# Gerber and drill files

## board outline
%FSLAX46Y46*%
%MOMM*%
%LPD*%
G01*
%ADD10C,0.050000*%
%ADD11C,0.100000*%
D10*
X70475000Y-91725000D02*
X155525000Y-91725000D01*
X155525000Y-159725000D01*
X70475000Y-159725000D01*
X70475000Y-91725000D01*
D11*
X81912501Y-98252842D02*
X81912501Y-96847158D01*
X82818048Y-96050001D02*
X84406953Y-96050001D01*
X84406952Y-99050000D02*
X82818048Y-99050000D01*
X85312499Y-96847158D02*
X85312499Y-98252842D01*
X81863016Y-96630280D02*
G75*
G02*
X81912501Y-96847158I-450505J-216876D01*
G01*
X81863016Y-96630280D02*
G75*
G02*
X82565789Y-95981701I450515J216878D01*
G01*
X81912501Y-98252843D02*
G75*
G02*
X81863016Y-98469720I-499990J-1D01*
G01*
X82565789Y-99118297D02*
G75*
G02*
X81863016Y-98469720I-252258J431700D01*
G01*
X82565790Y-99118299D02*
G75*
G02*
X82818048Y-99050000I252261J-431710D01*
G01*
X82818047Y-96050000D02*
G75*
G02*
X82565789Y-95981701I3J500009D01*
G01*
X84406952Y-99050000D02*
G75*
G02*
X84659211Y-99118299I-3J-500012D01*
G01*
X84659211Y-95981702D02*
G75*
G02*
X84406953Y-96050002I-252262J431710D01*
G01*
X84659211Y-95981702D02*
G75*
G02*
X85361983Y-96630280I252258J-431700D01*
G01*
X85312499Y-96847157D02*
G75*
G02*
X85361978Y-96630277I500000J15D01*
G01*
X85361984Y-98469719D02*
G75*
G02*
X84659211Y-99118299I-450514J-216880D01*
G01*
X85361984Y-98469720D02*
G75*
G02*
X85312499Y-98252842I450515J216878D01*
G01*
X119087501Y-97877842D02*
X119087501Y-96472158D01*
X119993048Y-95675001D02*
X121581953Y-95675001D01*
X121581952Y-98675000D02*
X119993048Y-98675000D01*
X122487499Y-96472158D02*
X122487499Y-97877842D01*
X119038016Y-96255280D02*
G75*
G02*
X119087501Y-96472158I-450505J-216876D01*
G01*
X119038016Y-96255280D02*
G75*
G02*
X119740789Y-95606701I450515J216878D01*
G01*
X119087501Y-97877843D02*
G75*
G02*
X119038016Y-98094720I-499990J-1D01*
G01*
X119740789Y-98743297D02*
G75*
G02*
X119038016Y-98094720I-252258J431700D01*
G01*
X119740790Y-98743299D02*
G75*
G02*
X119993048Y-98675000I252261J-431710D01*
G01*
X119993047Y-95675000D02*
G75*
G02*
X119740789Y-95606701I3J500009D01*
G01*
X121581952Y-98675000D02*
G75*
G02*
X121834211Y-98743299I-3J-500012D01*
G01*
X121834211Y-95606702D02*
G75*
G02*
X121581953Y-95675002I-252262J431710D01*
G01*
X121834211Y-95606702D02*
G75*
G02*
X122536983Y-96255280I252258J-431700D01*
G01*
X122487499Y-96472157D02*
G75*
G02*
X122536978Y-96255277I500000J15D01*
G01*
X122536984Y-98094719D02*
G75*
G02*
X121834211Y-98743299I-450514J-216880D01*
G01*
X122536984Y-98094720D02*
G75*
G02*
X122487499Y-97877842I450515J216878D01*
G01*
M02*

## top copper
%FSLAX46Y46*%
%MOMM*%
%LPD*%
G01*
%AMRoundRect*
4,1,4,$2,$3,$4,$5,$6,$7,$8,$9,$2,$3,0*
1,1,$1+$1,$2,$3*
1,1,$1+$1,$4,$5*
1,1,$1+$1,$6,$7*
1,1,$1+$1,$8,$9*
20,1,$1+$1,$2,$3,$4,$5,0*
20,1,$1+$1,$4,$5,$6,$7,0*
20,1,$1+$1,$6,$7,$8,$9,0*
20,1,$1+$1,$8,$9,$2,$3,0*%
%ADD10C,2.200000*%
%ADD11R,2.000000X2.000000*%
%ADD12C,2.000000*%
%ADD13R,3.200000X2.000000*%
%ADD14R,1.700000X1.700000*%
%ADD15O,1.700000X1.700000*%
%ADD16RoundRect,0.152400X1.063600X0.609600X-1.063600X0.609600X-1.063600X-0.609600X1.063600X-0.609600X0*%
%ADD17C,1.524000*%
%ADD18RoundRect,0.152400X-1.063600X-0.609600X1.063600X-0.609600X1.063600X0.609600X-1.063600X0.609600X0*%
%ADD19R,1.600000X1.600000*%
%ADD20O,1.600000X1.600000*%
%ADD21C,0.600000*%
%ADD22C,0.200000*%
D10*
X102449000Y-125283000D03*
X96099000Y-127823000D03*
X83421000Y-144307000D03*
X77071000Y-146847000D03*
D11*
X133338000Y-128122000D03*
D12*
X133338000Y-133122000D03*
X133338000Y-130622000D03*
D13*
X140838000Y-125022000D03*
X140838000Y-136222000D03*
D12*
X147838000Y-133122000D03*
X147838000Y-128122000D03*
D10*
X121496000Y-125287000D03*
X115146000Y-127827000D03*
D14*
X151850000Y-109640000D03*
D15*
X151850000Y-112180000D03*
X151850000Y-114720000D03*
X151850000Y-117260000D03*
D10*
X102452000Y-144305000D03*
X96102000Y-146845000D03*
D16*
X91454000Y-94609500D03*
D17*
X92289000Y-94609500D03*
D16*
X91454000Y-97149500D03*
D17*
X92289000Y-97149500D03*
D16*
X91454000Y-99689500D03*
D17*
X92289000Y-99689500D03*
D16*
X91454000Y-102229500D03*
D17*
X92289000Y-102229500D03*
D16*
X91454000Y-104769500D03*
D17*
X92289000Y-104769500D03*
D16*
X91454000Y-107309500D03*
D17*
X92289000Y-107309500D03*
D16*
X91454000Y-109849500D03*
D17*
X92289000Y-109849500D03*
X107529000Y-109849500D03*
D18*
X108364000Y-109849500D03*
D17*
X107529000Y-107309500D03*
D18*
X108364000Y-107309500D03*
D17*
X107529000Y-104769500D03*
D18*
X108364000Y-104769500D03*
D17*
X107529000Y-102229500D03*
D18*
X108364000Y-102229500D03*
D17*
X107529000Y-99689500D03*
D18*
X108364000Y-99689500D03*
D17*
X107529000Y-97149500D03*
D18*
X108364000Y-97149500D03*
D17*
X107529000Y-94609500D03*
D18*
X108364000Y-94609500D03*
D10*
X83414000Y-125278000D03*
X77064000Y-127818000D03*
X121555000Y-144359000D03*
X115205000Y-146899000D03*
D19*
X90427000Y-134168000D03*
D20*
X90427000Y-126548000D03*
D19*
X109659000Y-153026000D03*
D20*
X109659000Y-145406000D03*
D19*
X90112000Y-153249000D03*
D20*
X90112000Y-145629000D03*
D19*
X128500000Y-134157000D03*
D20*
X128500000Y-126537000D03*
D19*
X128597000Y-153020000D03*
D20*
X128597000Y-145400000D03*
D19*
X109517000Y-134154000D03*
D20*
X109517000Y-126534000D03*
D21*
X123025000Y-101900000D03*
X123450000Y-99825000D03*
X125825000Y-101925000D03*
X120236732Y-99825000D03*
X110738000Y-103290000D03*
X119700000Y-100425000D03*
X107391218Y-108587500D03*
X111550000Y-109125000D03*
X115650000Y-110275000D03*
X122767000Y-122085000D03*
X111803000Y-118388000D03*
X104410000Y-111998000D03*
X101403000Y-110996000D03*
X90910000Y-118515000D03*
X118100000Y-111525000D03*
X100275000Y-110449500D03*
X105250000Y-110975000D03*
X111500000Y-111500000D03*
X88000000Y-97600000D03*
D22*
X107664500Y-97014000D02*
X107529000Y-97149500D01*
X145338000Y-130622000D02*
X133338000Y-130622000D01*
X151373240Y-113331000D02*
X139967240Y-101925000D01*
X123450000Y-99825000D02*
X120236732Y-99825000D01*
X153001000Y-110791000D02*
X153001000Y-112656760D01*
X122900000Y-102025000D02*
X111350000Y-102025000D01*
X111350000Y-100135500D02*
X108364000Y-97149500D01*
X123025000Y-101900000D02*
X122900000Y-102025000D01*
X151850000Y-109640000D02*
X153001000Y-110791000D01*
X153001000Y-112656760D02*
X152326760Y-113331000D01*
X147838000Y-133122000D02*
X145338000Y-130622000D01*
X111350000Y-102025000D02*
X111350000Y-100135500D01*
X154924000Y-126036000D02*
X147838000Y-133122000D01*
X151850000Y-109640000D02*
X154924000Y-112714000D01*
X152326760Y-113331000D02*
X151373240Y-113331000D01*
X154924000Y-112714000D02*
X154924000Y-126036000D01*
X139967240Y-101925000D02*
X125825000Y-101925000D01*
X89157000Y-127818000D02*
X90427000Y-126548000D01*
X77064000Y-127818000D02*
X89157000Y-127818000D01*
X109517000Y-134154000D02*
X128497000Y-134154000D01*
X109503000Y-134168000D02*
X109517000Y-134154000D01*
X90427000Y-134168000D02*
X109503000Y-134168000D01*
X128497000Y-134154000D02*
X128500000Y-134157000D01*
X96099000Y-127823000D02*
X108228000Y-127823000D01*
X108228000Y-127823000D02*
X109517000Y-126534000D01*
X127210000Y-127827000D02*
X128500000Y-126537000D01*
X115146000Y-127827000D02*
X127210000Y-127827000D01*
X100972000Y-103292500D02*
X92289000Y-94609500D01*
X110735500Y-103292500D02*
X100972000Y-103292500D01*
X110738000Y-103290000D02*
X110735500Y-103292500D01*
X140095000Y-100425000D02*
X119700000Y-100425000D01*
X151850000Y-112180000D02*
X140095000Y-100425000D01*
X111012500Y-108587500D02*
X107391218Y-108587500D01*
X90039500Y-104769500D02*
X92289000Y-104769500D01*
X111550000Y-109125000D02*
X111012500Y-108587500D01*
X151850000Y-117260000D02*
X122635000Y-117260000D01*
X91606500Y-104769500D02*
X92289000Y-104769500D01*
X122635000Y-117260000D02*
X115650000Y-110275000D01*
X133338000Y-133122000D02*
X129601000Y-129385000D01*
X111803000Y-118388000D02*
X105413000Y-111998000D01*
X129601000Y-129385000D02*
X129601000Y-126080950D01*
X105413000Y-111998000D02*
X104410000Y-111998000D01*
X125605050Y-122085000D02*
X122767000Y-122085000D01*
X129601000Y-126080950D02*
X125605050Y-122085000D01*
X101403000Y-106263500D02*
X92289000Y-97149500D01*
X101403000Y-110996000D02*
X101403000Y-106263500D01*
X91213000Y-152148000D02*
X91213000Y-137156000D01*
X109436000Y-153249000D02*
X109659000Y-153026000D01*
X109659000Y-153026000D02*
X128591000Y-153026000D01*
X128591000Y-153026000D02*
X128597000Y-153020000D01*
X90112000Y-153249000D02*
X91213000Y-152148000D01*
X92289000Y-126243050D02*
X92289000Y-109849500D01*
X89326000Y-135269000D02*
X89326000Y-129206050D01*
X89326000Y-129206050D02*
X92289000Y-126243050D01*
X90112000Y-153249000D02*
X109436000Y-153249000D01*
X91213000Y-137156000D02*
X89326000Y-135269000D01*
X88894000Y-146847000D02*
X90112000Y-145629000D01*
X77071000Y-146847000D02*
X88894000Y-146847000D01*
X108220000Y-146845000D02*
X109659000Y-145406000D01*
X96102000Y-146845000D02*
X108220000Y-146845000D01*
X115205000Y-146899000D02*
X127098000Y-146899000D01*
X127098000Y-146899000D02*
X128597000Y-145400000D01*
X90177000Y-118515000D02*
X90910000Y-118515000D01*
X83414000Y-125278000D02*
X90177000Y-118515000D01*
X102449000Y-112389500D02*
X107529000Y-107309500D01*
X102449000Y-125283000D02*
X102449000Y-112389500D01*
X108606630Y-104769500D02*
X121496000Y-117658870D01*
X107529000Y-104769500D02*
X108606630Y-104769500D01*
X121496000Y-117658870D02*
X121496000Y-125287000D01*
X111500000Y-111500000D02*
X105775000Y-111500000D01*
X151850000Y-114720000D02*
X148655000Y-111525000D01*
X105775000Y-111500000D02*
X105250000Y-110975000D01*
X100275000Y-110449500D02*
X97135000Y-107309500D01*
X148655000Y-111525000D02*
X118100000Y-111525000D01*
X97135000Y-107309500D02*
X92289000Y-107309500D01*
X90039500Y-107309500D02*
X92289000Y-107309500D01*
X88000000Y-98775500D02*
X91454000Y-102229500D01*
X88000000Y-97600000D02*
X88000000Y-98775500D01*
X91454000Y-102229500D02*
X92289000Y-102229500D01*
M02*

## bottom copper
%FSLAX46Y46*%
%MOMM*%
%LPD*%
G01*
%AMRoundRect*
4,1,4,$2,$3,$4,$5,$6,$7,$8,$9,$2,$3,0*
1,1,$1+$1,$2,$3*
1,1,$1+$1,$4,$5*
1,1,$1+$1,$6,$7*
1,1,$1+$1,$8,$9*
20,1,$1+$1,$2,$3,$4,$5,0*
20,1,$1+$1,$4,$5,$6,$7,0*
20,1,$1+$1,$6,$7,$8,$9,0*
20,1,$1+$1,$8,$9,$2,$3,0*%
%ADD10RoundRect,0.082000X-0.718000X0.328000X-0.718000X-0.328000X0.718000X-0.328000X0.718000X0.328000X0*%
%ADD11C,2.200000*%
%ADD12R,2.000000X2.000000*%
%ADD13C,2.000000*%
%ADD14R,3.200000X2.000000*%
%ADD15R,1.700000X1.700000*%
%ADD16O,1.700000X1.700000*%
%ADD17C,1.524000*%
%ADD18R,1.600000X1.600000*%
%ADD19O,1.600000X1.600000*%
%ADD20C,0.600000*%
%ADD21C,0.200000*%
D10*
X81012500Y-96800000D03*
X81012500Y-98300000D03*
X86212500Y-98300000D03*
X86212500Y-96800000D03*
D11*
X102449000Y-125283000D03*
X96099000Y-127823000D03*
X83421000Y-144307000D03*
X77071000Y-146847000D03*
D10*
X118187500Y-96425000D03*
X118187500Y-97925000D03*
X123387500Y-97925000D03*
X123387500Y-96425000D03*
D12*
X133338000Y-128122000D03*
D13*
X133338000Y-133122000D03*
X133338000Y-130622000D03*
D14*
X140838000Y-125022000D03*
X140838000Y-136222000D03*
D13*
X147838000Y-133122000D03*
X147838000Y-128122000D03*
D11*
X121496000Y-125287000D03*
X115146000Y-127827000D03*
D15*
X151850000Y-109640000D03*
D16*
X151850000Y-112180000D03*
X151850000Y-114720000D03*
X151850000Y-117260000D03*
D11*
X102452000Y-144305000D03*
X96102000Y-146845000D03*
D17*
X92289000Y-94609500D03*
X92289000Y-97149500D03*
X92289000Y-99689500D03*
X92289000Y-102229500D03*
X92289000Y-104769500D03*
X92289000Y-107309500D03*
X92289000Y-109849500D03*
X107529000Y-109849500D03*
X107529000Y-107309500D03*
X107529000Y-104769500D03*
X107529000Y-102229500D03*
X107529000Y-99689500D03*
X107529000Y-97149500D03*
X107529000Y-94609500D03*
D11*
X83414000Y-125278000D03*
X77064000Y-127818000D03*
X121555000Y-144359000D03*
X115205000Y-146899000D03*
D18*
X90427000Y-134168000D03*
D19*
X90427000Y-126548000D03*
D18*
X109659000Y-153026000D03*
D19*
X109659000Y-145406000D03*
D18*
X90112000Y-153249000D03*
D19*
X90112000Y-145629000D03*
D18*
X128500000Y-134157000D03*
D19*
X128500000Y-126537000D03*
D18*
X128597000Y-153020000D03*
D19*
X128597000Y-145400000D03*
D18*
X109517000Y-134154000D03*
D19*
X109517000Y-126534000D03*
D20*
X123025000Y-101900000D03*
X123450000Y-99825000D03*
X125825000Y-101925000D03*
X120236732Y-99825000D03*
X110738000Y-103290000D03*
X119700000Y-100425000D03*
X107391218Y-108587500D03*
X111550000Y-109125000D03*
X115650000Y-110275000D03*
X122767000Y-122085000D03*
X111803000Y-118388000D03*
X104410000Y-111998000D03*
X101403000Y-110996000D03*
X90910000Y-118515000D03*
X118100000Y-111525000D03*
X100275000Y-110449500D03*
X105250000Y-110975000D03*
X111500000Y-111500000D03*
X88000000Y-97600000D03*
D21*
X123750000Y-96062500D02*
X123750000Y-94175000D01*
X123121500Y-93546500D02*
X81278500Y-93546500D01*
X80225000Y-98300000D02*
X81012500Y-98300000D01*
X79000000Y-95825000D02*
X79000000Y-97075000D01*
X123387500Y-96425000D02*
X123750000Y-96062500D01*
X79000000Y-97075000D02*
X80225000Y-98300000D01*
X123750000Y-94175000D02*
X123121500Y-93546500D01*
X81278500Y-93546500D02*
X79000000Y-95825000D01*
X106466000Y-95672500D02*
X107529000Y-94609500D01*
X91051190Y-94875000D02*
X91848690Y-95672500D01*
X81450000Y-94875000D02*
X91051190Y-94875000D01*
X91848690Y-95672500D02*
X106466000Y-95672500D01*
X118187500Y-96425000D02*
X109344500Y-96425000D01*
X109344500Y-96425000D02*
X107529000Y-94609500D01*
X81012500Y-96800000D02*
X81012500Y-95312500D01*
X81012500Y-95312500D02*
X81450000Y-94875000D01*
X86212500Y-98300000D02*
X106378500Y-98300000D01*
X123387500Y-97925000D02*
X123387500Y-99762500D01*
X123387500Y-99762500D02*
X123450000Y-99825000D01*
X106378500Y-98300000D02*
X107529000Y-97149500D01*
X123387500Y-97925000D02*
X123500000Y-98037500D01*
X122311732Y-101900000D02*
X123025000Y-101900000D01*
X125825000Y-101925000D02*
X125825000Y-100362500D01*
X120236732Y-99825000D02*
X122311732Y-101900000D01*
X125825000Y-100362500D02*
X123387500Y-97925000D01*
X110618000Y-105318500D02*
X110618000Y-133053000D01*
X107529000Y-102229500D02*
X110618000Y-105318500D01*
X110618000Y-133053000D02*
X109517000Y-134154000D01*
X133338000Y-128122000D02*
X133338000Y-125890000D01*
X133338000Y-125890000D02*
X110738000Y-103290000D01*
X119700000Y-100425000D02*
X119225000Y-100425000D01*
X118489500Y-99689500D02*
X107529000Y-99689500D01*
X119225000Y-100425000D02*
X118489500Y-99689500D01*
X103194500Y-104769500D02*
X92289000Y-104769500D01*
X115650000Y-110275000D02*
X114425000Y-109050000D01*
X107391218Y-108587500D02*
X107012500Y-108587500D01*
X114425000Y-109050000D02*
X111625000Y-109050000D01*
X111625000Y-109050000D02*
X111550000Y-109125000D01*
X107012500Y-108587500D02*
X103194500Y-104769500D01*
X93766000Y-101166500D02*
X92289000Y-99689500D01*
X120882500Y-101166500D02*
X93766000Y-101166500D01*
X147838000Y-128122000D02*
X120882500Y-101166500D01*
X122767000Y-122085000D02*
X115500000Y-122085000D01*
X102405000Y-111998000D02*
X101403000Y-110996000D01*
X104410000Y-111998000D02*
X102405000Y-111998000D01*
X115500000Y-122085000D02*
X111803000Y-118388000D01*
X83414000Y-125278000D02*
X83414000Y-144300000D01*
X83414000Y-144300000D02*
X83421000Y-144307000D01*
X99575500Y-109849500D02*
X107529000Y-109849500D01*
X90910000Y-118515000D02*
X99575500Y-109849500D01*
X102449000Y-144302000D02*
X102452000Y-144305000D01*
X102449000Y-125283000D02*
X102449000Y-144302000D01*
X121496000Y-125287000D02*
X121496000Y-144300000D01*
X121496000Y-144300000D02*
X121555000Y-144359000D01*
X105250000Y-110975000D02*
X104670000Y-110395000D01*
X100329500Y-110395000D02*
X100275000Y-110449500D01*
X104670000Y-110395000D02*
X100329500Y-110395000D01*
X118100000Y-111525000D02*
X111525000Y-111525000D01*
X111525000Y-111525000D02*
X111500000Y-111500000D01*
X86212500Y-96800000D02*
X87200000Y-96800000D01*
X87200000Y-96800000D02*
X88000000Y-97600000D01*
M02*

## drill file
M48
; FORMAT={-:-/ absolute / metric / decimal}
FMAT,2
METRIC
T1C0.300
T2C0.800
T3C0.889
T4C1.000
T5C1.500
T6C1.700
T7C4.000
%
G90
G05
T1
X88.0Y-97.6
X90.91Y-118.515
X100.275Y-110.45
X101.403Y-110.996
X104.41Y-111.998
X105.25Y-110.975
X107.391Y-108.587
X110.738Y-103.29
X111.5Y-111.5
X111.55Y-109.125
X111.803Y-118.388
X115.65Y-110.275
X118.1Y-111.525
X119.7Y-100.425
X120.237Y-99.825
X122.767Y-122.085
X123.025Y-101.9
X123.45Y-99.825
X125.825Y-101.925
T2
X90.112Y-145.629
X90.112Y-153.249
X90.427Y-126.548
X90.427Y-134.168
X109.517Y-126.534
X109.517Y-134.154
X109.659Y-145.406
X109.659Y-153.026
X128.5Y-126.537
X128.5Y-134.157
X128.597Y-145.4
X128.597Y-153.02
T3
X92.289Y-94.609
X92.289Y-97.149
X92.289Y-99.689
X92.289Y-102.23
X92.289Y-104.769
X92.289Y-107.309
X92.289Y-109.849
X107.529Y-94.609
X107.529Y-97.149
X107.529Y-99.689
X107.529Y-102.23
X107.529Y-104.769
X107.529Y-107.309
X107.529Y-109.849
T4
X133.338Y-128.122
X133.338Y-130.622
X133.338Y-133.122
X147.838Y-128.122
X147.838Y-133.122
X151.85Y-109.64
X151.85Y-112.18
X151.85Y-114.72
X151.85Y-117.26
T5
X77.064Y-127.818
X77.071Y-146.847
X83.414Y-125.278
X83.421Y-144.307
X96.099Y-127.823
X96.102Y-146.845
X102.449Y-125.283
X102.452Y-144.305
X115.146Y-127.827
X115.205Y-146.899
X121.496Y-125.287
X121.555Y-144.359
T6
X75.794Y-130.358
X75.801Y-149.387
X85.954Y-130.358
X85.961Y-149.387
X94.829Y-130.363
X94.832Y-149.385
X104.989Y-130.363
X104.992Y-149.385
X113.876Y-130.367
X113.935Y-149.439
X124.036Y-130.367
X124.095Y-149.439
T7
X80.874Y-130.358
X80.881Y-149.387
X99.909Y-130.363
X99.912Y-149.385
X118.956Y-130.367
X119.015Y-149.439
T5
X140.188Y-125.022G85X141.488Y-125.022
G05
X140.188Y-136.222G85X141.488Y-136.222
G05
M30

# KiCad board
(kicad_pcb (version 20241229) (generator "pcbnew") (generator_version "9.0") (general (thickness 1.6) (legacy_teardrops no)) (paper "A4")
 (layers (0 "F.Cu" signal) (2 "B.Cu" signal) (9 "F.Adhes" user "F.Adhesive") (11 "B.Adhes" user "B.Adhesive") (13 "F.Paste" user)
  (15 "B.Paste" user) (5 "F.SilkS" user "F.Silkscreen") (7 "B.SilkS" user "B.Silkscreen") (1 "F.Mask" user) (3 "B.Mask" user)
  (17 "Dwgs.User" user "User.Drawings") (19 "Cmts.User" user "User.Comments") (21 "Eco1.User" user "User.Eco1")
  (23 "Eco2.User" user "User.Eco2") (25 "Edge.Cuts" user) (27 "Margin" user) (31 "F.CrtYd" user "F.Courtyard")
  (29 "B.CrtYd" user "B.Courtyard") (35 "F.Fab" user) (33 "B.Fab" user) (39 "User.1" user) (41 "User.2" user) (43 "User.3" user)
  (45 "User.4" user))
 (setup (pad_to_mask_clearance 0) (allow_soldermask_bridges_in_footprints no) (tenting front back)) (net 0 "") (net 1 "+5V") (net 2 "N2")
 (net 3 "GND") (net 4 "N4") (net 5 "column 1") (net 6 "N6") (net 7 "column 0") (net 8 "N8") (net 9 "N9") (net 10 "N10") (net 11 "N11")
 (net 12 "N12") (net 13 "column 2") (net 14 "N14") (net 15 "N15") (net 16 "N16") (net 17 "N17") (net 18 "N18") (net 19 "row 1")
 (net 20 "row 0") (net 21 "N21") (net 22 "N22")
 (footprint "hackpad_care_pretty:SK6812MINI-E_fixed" (layer "F.Cu") (at 83.612499 97.652842)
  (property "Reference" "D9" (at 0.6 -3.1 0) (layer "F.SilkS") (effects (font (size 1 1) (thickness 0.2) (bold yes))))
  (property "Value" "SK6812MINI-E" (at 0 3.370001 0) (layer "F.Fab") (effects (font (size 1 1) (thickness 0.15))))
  (fp_line (start -1.699998 0.6) (end -1.699998 -0.805684) (stroke (width 0.1) (type solid)) (layer "Edge.Cuts"))
  (fp_line (start -0.794451 -1.602841) (end 0.794454 -1.602841) (stroke (width 0.1) (type solid)) (layer "Edge.Cuts"))
  (fp_line (start 0.794453 1.397158) (end -0.794451 1.397158) (stroke (width 0.1) (type solid)) (layer "Edge.Cuts"))
  (fp_line (start 1.7 -0.805684) (end 1.7 0.6) (stroke (width 0.1) (type solid)) (layer "Edge.Cuts"))
  (fp_arc (start -1.749483 -1.022562) (mid -1.712526 -0.91691) (end -1.699998 -0.805684) (stroke (width 0.1) (type solid))
   (layer "Edge.Cuts"))
  (fp_arc (start -1.749483 -1.022562) (mid -1.63807 -1.606877) (end -1.04671 -1.671141) (stroke (width 0.1) (type solid))
   (layer "Edge.Cuts"))
  (fp_arc (start -1.699998 0.600001) (mid -1.712526 0.711226) (end -1.749483 0.816878) (stroke (width 0.1) (type solid)) (layer "Edge.Cuts"))
  (fp_arc (start -1.04671 1.465455) (mid -1.638069 1.401192) (end -1.749483 0.816878) (stroke (width 0.1) (type solid)) (layer "Edge.Cuts"))
  (fp_arc (start -1.046709 1.465457) (mid -0.925121 1.414535) (end -0.794451 1.397158) (stroke (width 0.1) (type solid)) (layer "Edge.Cuts"))
  (fp_arc (start -0.794452 -1.602842) (mid -0.925122 -1.620219) (end -1.04671 -1.671141) (stroke (width 0.1) (type solid))
   (layer "Edge.Cuts"))
  (fp_arc (start 0.794453 1.397158) (mid 0.925124 1.414535) (end 1.046712 1.465457) (stroke (width 0.1) (type solid)) (layer "Edge.Cuts"))
  (fp_arc (start 1.046712 -1.67114) (mid 0.925124 -1.620218) (end 0.794454 -1.602841) (stroke (width 0.1) (type solid)) (layer "Edge.Cuts"))
  (fp_arc (start 1.046712 -1.67114) (mid 1.638072 -1.606876) (end 1.749485 -1.022562) (stroke (width 0.1) (type solid)) (layer "Edge.Cuts"))
  (fp_arc (start 1.7 -0.805685) (mid 1.712528 -0.91691) (end 1.749485 -1.022562) (stroke (width 0.1) (type solid)) (layer "Edge.Cuts"))
  (fp_arc (start 1.749485 0.816877) (mid 1.638073 1.401193) (end 1.046712 1.465457) (stroke (width 0.1) (type solid)) (layer "Edge.Cuts"))
  (fp_arc (start 1.749485 0.816878) (mid 1.712528 0.711226) (end 1.7 0.6) (stroke (width 0.1) (type solid)) (layer "Edge.Cuts"))
  (pad "1" smd roundrect (at -2.599999 -0.852842 270) (size 0.82 1.6) (layers "B.Cu" "B.Mask" "B.Paste") (roundrect_rratio 0.1)
   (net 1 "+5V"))
  (pad "2" smd roundrect (at -2.599999 0.647158 270) (size 0.82 1.6) (layers "B.Cu" "B.Mask" "B.Paste") (roundrect_rratio 0.1) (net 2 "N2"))
  (pad "3" smd roundrect (at 2.600001 0.647158 270) (size 0.82 1.6) (layers "B.Cu" "B.Mask" "B.Paste") (roundrect_rratio 0.1) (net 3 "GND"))
  (pad "4" smd roundrect (at 2.600001 -0.852842 270) (size 0.82 1.6) (layers "B.Cu" "B.Mask" "B.Paste") (roundrect_rratio 0.1) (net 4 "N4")))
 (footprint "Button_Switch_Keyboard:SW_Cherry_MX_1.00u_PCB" (layer "F.Cu") (at 102.449 125.283)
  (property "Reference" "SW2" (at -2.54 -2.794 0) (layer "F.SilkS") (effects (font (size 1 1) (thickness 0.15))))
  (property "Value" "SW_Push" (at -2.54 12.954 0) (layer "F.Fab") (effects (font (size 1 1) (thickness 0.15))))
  (pad "" np_thru_hole circle (at -7.62 5.08) (size 1.7 1.7) (drill 1.7) (layers "*.Cu" "*.Mask"))
  (pad "" np_thru_hole circle (at -2.54 5.08) (size 4 4) (drill 4) (layers "*.Cu" "*.Mask"))
  (pad "" np_thru_hole circle (at 2.54 5.08) (size 1.7 1.7) (drill 1.7) (layers "*.Cu" "*.Mask"))
  (pad "1" thru_hole circle (at 0 0) (size 2.2 2.2) (drill 1.5) (layers "*.Cu" "*.Mask") (remove_unused_layers no) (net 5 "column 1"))
  (pad "2" thru_hole circle (at -6.35 2.54) (size 2.2 2.2) (drill 1.5) (layers "*.Cu" "*.Mask") (remove_unused_layers no) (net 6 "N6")))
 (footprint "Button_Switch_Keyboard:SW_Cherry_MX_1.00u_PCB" (layer "F.Cu") (at 83.421 144.307)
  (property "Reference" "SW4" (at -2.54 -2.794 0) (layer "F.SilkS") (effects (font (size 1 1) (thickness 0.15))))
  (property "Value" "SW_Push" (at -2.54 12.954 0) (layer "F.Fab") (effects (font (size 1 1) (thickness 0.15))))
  (pad "" np_thru_hole circle (at -7.62 5.08) (size 1.7 1.7) (drill 1.7) (layers "*.Cu" "*.Mask"))
  (pad "" np_thru_hole circle (at -2.54 5.08) (size 4 4) (drill 4) (layers "*.Cu" "*.Mask"))
  (pad "" np_thru_hole circle (at 2.54 5.08) (size 1.7 1.7) (drill 1.7) (layers "*.Cu" "*.Mask"))
  (pad "1" thru_hole circle (at 0 0) (size 2.2 2.2) (drill 1.5) (layers "*.Cu" "*.Mask") (remove_unused_layers no) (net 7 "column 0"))
  (pad "2" thru_hole circle (at -6.35 2.54) (size 2.2 2.2) (drill 1.5) (layers "*.Cu" "*.Mask") (remove_unused_layers no) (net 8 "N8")))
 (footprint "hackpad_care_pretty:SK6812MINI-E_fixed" (layer "F.Cu") (at 120.787499 97.277842)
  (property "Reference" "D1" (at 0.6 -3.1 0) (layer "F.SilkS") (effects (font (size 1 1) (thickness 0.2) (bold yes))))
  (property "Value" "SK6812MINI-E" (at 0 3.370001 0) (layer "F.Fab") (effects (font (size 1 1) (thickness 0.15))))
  (fp_line (start -1.699998 0.6) (end -1.699998 -0.805684) (stroke (width 0.1) (type solid)) (layer "Edge.Cuts"))
  (fp_line (start -0.794451 -1.602841) (end 0.794454 -1.602841) (stroke (width 0.1) (type solid)) (layer "Edge.Cuts"))
  (fp_line (start 0.794453 1.397158) (end -0.794451 1.397158) (stroke (width 0.1) (type solid)) (layer "Edge.Cuts"))
  (fp_line (start 1.7 -0.805684) (end 1.7 0.6) (stroke (width 0.1) (type solid)) (layer "Edge.Cuts"))
  (fp_arc (start -1.749483 -1.022562) (mid -1.712526 -0.91691) (end -1.699998 -0.805684) (stroke (width 0.1) (type solid))
   (layer "Edge.Cuts"))
  (fp_arc (start -1.749483 -1.022562) (mid -1.63807 -1.606877) (end -1.04671 -1.671141) (stroke (width 0.1) (type solid))
   (layer "Edge.Cuts"))
  (fp_arc (start -1.699998 0.600001) (mid -1.712526 0.711226) (end -1.749483 0.816878) (stroke (width 0.1) (type solid)) (layer "Edge.Cuts"))
  (fp_arc (start -1.04671 1.465455) (mid -1.638069 1.401192) (end -1.749483 0.816878) (stroke (width 0.1) (type solid)) (layer "Edge.Cuts"))
  (fp_arc (start -1.046709 1.465457) (mid -0.925121 1.414535) (end -0.794451 1.397158) (stroke (width 0.1) (type solid)) (layer "Edge.Cuts"))
  (fp_arc (start -0.794452 -1.602842) (mid -0.925122 -1.620219) (end -1.04671 -1.671141) (stroke (width 0.1) (type solid))
   (layer "Edge.Cuts"))
  (fp_arc (start 0.794453 1.397158) (mid 0.925124 1.414535) (end 1.046712 1.465457) (stroke (width 0.1) (type solid)) (layer "Edge.Cuts"))
  (fp_arc (start 1.046712 -1.67114) (mid 0.925124 -1.620218) (end 0.794454 -1.602841) (stroke (width 0.1) (type solid)) (layer "Edge.Cuts"))
  (fp_arc (start 1.046712 -1.67114) (mid 1.638072 -1.606876) (end 1.749485 -1.022562) (stroke (width 0.1) (type solid)) (layer "Edge.Cuts"))
  (fp_arc (start 1.7 -0.805685) (mid 1.712528 -0.91691) (end 1.749485 -1.022562) (stroke (width 0.1) (type solid)) (layer "Edge.Cuts"))
  (fp_arc (start 1.749485 0.816877) (mid 1.638073 1.401193) (end 1.046712 1.465457) (stroke (width 0.1) (type solid)) (layer "Edge.Cuts"))
  (fp_arc (start 1.749485 0.816878) (mid 1.712528 0.711226) (end 1.7 0.6) (stroke (width 0.1) (type solid)) (layer "Edge.Cuts"))
  (pad "1" smd roundrect (at -2.599999 -0.852842 270) (size 0.82 1.6) (layers "B.Cu" "B.Mask" "B.Paste") (roundrect_rratio 0.1)
   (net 1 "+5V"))
  (pad "2" smd roundrect (at -2.599999 0.647158 270) (size 0.82 1.6) (layers "B.Cu" "B.Mask" "B.Paste") (roundrect_rratio 0.1) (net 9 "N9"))
  (pad "3" smd roundrect (at 2.600001 0.647158 270) (size 0.82 1.6) (layers "B.Cu" "B.Mask" "B.Paste") (roundrect_rratio 0.1) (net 3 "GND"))
  (pad "4" smd roundrect (at 2.600001 -0.852842 270) (size 0.82 1.6) (layers "B.Cu" "B.Mask" "B.Paste") (roundrect_rratio 0.1) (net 2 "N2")))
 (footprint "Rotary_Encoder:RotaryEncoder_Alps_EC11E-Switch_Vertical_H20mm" (layer "F.Cu") (at 133.338 128.122)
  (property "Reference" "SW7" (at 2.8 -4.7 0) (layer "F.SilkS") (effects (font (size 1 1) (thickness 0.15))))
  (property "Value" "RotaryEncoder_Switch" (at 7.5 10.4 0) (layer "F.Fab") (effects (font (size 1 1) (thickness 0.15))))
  (pad "A" thru_hole rect (at 0 0) (size 2 2) (drill 1) (layers "*.Cu" "*.Mask") (remove_unused_layers no) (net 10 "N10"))
  (pad "B" thru_hole circle (at 0 5) (size 2 2) (drill 1) (layers "*.Cu" "*.Mask") (remove_unused_layers no) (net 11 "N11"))
  (pad "C" thru_hole circle (at 0 2.5) (size 2 2) (drill 1) (layers "*.Cu" "*.Mask") (remove_unused_layers no) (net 3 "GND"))
  (pad "MP" thru_hole rect (at 7.5 -3.1) (size 3.2 2) (drill oval 2.8 1.5) (layers "*.Cu" "*.Mask") (remove_unused_layers no))
  (pad "MP" thru_hole rect (at 7.5 8.1) (size 3.2 2) (drill oval 2.8 1.5) (layers "*.Cu" "*.Mask") (remove_unused_layers no))
  (pad "S1" thru_hole circle (at 14.5 5) (size 2 2) (drill 1) (layers "*.Cu" "*.Mask") (remove_unused_layers no) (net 3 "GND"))
  (pad "S2" thru_hole circle (at 14.5 0) (size 2 2) (drill 1) (layers "*.Cu" "*.Mask") (remove_unused_layers no) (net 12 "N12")))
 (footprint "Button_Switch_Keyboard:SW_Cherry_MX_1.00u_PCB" (layer "F.Cu") (at 121.496 125.287)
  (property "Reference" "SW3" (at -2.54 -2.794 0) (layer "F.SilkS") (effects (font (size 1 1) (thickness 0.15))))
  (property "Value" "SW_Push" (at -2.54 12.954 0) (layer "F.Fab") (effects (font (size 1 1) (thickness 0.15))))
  (pad "" np_thru_hole circle (at -7.62 5.08) (size 1.7 1.7) (drill 1.7) (layers "*.Cu" "*.Mask"))
  (pad "" np_thru_hole circle (at -2.54 5.08) (size 4 4) (drill 4) (layers "*.Cu" "*.Mask"))
  (pad "" np_thru_hole circle (at 2.54 5.08) (size 1.7 1.7) (drill 1.7) (layers "*.Cu" "*.Mask"))
  (pad "1" thru_hole circle (at 0 0) (size 2.2 2.2) (drill 1.5) (layers "*.Cu" "*.Mask") (remove_unused_layers no) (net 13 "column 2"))
  (pad "2" thru_hole circle (at -6.35 2.54) (size 2.2 2.2) (drill 1.5) (layers "*.Cu" "*.Mask") (remove_unused_layers no) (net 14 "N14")))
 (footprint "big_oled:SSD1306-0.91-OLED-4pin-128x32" (layer "F.Cu") (at 115.35 107.45)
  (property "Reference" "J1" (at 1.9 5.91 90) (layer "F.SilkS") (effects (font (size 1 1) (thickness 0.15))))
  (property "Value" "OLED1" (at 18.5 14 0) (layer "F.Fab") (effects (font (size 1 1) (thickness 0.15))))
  (pad "1" thru_hole rect (at 36.5 2.19) (size 1.7 1.7) (drill 1) (layers "*.Cu" "*.Mask") (remove_unused_layers no) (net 3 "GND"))
  (pad "2" thru_hole oval (at 36.5 4.73) (size 1.7 1.7) (drill 1) (layers "*.Cu" "*.Mask") (remove_unused_layers no) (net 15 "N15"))
  (pad "3" thru_hole oval (at 36.5 7.27) (size 1.7 1.7) (drill 1) (layers "*.Cu" "*.Mask") (remove_unused_layers no) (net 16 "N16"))
  (pad "4" thru_hole oval (at 36.5 9.81) (size 1.7 1.7) (drill 1) (layers "*.Cu" "*.Mask") (remove_unused_layers no) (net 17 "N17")))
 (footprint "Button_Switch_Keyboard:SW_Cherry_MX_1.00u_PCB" (layer "F.Cu") (at 102.452 144.305)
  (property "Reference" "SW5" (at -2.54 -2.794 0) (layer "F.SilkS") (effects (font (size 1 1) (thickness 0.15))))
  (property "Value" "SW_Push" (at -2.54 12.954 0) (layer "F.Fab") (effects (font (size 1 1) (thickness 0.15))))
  (pad "" np_thru_hole circle (at -7.62 5.08) (size 1.7 1.7) (drill 1.7) (layers "*.Cu" "*.Mask"))
  (pad "" np_thru_hole circle (at -2.54 5.08) (size 4 4) (drill 4) (layers "*.Cu" "*.Mask"))
  (pad "" np_thru_hole circle (at 2.54 5.08) (size 1.7 1.7) (drill 1.7) (layers "*.Cu" "*.Mask"))
  (pad "1" thru_hole circle (at 0 0) (size 2.2 2.2) (drill 1.5) (layers "*.Cu" "*.Mask") (remove_unused_layers no) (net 5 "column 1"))
  (pad "2" thru_hole circle (at -6.35 2.54) (size 2.2 2.2) (drill 1.5) (layers "*.Cu" "*.Mask") (remove_unused_layers no) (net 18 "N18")))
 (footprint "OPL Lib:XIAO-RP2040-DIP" (layer "F.Cu") (at 99.909 102.2295)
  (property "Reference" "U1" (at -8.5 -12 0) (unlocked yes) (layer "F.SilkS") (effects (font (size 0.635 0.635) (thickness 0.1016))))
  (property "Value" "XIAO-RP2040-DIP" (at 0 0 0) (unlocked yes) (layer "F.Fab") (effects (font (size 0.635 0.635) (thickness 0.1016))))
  (pad "1" smd roundrect (at -8.455 -7.62 180) (size 2.432 1.524) (layers "F.Cu" "F.Mask") (roundrect_rratio 0.1) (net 10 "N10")
   (thermal_bridge_angle 45))
  (pad "1" thru_hole circle (at -7.62 -7.62 180) (size 1.524 1.524) (drill 0.889) (layers "*.Cu" "*.Mask") (remove_unused_layers no)
   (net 10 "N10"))
  (pad "2" smd roundrect (at -8.455 -5.08 180) (size 2.432 1.524) (layers "F.Cu" "F.Mask") (roundrect_rratio 0.1) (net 11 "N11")
   (thermal_bridge_angle 45))
  (pad "2" thru_hole circle (at -7.62 -5.08 180) (size 1.524 1.524) (drill 0.889) (layers "*.Cu" "*.Mask") (remove_unused_layers no)
   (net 11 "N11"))
  (pad "3" smd roundrect (at -8.455 -2.54 180) (size 2.432 1.524) (layers "F.Cu" "F.Mask") (roundrect_rratio 0.1) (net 12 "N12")
   (thermal_bridge_angle 45))
  (pad "3" thru_hole circle (at -7.62 -2.54 180) (size 1.524 1.524) (drill 0.889) (layers "*.Cu" "*.Mask") (remove_unused_layers no)
   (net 12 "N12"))
  (pad "4" smd roundrect (at -8.455 0 180) (size 2.432 1.524) (layers "F.Cu" "F.Mask") (roundrect_rratio 0.1) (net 4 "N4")
   (thermal_bridge_angle 45))
  (pad "4" thru_hole circle (at -7.62 0 180) (size 1.524 1.524) (drill 0.889) (layers "*.Cu" "*.Mask") (remove_unused_layers no)
   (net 4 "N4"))
  (pad "5" smd roundrect (at -8.455 2.54 180) (size 2.432 1.524) (layers "F.Cu" "F.Mask") (roundrect_rratio 0.1) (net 17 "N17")
   (thermal_bridge_angle 45))
  (pad "5" thru_hole circle (at -7.62 2.54 180) (size 1.524 1.524) (drill 0.889) (layers "*.Cu" "*.Mask") (remove_unused_layers no)
   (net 17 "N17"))
  (pad "6" smd roundrect (at -8.455 5.08 180) (size 2.432 1.524) (layers "F.Cu" "F.Mask") (roundrect_rratio 0.1) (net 16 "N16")
   (thermal_bridge_angle 45))
  (pad "6" thru_hole circle (at -7.62 5.08 180) (size 1.524 1.524) (drill 0.889) (layers "*.Cu" "*.Mask") (remove_unused_layers no)
   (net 16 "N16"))
  (pad "7" smd roundrect (at -8.455 7.62 180) (size 2.432 1.524) (layers "F.Cu" "F.Mask") (roundrect_rratio 0.1) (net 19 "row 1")
   (thermal_bridge_angle 45))
  (pad "7" thru_hole circle (at -7.62 7.62 180) (size 1.524 1.524) (drill 0.889) (layers "*.Cu" "*.Mask") (remove_unused_layers no)
   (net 19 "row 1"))
  (pad "8" thru_hole circle (at 7.62 7.62) (size 1.524 1.524) (drill 0.889) (layers "*.Cu" "*.Mask") (remove_unused_layers no)
   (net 7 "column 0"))
  (pad "8" smd roundrect (at 8.455 7.62) (size 2.432 1.524) (layers "F.Cu" "F.Mask") (roundrect_rratio 0.1) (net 7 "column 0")
   (thermal_bridge_angle 45))
  (pad "9" thru_hole circle (at 7.62 5.08) (size 1.524 1.524) (drill 0.889) (layers "*.Cu" "*.Mask") (remove_unused_layers no)
   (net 5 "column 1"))
  (pad "9" smd roundrect (at 8.455 5.08) (size 2.432 1.524) (layers "F.Cu" "F.Mask") (roundrect_rratio 0.1) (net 5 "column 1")
   (thermal_bridge_angle 45))
  (pad "10" thru_hole circle (at 7.62 2.54) (size 1.524 1.524) (drill 0.889) (layers "*.Cu" "*.Mask") (remove_unused_layers no)
   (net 13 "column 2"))
  (pad "10" smd roundrect (at 8.455 2.54) (size 2.432 1.524) (layers "F.Cu" "F.Mask") (roundrect_rratio 0.1) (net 13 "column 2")
   (thermal_bridge_angle 45))
  (pad "11" thru_hole circle (at 7.62 0) (size 1.524 1.524) (drill 0.889) (layers "*.Cu" "*.Mask") (remove_unused_layers no)
   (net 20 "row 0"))
  (pad "11" smd roundrect (at 8.455 0) (size 2.432 1.524) (layers "F.Cu" "F.Mask") (roundrect_rratio 0.1) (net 20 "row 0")
   (thermal_bridge_angle 45))
  (pad "12" thru_hole circle (at 7.62 -2.54) (size 1.524 1.524) (drill 0.889) (layers "*.Cu" "*.Mask") (remove_unused_layers no)
   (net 15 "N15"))
  (pad "12" smd roundrect (at 8.455 -2.54) (size 2.432 1.524) (layers "F.Cu" "F.Mask") (roundrect_rratio 0.1) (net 15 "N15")
   (thermal_bridge_angle 45))
  (pad "13" thru_hole circle (at 7.62 -5.08) (size 1.524 1.524) (drill 0.889) (layers "*.Cu" "*.Mask") (remove_unused_layers no)
   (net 3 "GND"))
  (pad "13" smd roundrect (at 8.455 -5.08) (size 2.432 1.524) (layers "F.Cu" "F.Mask") (roundrect_rratio 0.1) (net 3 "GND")
   (thermal_bridge_angle 45))
  (pad "14" thru_hole circle (at 7.62 -7.62) (size 1.524 1.524) (drill 0.889) (layers "*.Cu" "*.Mask") (remove_unused_layers no)
   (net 1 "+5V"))
  (pad "14" smd roundrect (at 8.455 -7.62) (size 2.432 1.524) (layers "F.Cu" "F.Mask") (roundrect_rratio 0.1) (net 1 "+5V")
   (thermal_bridge_angle 45)))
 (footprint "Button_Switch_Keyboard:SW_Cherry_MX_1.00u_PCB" (layer "F.Cu") (at 83.414 125.278)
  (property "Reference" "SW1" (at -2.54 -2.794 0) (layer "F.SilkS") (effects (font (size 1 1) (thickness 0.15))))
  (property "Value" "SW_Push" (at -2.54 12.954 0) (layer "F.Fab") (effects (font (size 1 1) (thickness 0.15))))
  (pad "" np_thru_hole circle (at -7.62 5.08) (size 1.7 1.7) (drill 1.7) (layers "*.Cu" "*.Mask"))
  (pad "" np_thru_hole circle (at -2.54 5.08) (size 4 4) (drill 4) (layers "*.Cu" "*.Mask"))
  (pad "" np_thru_hole circle (at 2.54 5.08) (size 1.7 1.7) (drill 1.7) (layers "*.Cu" "*.Mask"))
  (pad "1" thru_hole circle (at 0 0) (size 2.2 2.2) (drill 1.5) (layers "*.Cu" "*.Mask") (remove_unused_layers no) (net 7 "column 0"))
  (pad "2" thru_hole circle (at -6.35 2.54) (size 2.2 2.2) (drill 1.5) (layers "*.Cu" "*.Mask") (remove_unused_layers no) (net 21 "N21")))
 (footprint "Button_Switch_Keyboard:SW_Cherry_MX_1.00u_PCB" (layer "F.Cu") (at 121.555 144.359)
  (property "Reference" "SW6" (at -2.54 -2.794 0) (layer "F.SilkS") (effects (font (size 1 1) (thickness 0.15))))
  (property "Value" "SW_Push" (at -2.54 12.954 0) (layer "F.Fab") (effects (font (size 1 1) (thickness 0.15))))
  (pad "" np_thru_hole circle (at -7.62 5.08) (size 1.7 1.7) (drill 1.7) (layers "*.Cu" "*.Mask"))
  (pad "" np_thru_hole circle (at -2.54 5.08) (size 4 4) (drill 4) (layers "*.Cu" "*.Mask"))
  (pad "" np_thru_hole circle (at 2.54 5.08) (size 1.7 1.7) (drill 1.7) (layers "*.Cu" "*.Mask"))
  (pad "1" thru_hole circle (at 0 0) (size 2.2 2.2) (drill 1.5) (layers "*.Cu" "*.Mask") (remove_unused_layers no) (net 13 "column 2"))
  (pad "2" thru_hole circle (at -6.35 2.54) (size 2.2 2.2) (drill 1.5) (layers "*.Cu" "*.Mask") (remove_unused_layers no) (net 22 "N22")))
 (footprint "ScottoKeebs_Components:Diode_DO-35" (layer "B.Cu") (at 90.427 134.168 90)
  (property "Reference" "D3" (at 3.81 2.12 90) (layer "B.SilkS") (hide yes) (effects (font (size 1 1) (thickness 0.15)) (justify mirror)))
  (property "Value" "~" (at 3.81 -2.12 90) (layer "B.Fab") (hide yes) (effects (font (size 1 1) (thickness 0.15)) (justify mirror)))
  (pad "1" thru_hole rect (at 0 0 90) (size 1.6 1.6) (drill 0.8) (layers "*.Cu" "*.Mask") (remove_unused_layers no) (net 20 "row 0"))
  (pad "2" thru_hole oval (at 7.62 0 90) (size 1.6 1.6) (drill 0.8) (layers "*.Cu" "*.Mask") (remove_unused_layers no) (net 21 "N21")))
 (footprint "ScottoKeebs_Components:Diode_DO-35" (layer "B.Cu") (at 109.659 153.026 90)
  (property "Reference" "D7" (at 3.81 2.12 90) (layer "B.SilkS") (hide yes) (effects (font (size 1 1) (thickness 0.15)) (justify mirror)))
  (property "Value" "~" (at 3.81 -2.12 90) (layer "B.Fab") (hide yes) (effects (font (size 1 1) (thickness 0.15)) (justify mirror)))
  (pad "1" thru_hole rect (at 0 0 90) (size 1.6 1.6) (drill 0.8) (layers "*.Cu" "*.Mask") (remove_unused_layers no) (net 19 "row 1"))
  (pad "2" thru_hole oval (at 7.62 0 90) (size 1.6 1.6) (drill 0.8) (layers "*.Cu" "*.Mask") (remove_unused_layers no) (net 18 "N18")))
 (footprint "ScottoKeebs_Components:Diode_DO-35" (layer "B.Cu") (at 90.112 153.249 90)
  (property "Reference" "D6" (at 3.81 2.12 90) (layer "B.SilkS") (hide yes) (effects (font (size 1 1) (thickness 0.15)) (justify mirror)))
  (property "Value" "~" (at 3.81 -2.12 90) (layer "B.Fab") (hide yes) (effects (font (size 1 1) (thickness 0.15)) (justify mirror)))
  (pad "1" thru_hole rect (at 0 0 90) (size 1.6 1.6) (drill 0.8) (layers "*.Cu" "*.Mask") (remove_unused_layers no) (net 19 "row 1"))
  (pad "2" thru_hole oval (at 7.62 0 90) (size 1.6 1.6) (drill 0.8) (layers "*.Cu" "*.Mask") (remove_unused_layers no) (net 8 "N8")))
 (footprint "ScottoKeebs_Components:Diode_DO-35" (layer "B.Cu") (at 128.5 134.157 90)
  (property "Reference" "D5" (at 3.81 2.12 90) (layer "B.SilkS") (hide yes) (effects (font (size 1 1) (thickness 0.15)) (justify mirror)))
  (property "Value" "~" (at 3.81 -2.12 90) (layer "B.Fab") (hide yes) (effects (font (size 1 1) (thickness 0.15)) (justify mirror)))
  (pad "1" thru_hole rect (at 0 0 90) (size 1.6 1.6) (drill 0.8) (layers "*.Cu" "*.Mask") (remove_unused_layers no) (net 20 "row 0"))
  (pad "2" thru_hole oval (at 7.62 0 90) (size 1.6 1.6) (drill 0.8) (layers "*.Cu" "*.Mask") (remove_unused_layers no) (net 14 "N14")))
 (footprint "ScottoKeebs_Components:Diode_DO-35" (layer "B.Cu") (at 128.597 153.02 90)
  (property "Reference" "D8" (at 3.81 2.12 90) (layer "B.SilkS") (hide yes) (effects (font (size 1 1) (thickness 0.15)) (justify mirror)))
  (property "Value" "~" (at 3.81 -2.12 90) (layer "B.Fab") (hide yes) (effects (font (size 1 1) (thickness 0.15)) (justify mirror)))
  (pad "1" thru_hole rect (at 0 0 90) (size 1.6 1.6) (drill 0.8) (layers "*.Cu" "*.Mask") (remove_unused_layers no) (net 19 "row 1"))
  (pad "2" thru_hole oval (at 7.62 0 90) (size 1.6 1.6) (drill 0.8) (layers "*.Cu" "*.Mask") (remove_unused_layers no) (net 22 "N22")))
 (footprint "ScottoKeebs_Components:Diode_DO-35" (layer "B.Cu") (at 109.517 134.154 90)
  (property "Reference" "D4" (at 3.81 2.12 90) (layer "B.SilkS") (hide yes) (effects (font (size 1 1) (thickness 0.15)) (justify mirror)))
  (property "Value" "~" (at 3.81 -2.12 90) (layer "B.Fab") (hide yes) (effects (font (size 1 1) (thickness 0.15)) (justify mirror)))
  (pad "1" thru_hole rect (at 0 0 90) (size 1.6 1.6) (drill 0.8) (layers "*.Cu" "*.Mask") (remove_unused_layers no) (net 20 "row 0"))
  (pad "2" thru_hole oval (at 7.62 0 90) (size 1.6 1.6) (drill 0.8) (layers "*.Cu" "*.Mask") (remove_unused_layers no) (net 6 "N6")))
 (gr_rect (start 70.475 91.725) (end 155.525 159.725) (stroke (width 0.05) (type default)) (fill no) (layer "Edge.Cuts"))
 (segment (start 123.75 96.0625) (end 123.75 94.175) (width 0.2) (layer "B.Cu") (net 2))
 (segment (start 123.1215 93.5465) (end 81.2785 93.5465) (width 0.2) (layer "B.Cu") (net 2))
 (segment (start 80.225 98.3) (end 81.0125 98.3) (width 0.2) (layer "B.Cu") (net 2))
 (segment (start 79 95.825) (end 79 97.075) (width 0.2) (layer "B.Cu") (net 2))
 (segment (start 123.3875 96.425) (end 123.75 96.0625) (width 0.2) (layer "B.Cu") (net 2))
 (segment (start 79 97.075) (end 80.225 98.3) (width 0.2) (layer "B.Cu") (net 2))
 (segment (start 123.75 94.175) (end 123.1215 93.5465) (width 0.2) (layer "B.Cu") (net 2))
 (segment (start 81.2785 93.5465) (end 79 95.825) (width 0.2) (layer "B.Cu") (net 2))
 (segment (start 106.466 95.6725) (end 107.529 94.6095) (width 0.2) (layer "B.Cu") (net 1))
 (segment (start 91.05119 94.875) (end 91.84869 95.6725) (width 0.2) (layer "B.Cu") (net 1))
 (segment (start 81.45 94.875) (end 91.05119 94.875) (width 0.2) (layer "B.Cu") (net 1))
 (segment (start 91.84869 95.6725) (end 106.466 95.6725) (width 0.2) (layer "B.Cu") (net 1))
 (segment (start 118.1875 96.425) (end 109.3445 96.425) (width 0.2) (layer "B.Cu") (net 1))
 (segment (start 109.3445 96.425) (end 107.529 94.6095) (width 0.2) (layer "B.Cu") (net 1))
 (segment (start 81.0125 96.8) (end 81.0125 95.3125) (width 0.2) (layer "B.Cu") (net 1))
 (segment (start 81.0125 95.3125) (end 81.45 94.875) (width 0.2) (layer "B.Cu") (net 1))
 (segment (start 107.6645 97.014) (end 107.529 97.1495) (width 0.2) (layer "F.Cu") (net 3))
 (segment (start 145.338 130.622) (end 133.338 130.622) (width 0.2) (layer "F.Cu") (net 3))
 (segment (start 151.37324 113.331) (end 139.96724 101.925) (width 0.2) (layer "F.Cu") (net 3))
 (segment (start 123.45 99.825) (end 120.236732 99.825) (width 0.2) (layer "F.Cu") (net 3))
 (segment (start 153.001 110.791) (end 153.001 112.65676) (width 0.2) (layer "F.Cu") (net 3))
 (segment (start 122.9 102.025) (end 111.35 102.025) (width 0.2) (layer "F.Cu") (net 3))
 (segment (start 111.35 100.1355) (end 108.364 97.1495) (width 0.2) (layer "F.Cu") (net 3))
 (segment (start 123.025 101.9) (end 122.9 102.025) (width 0.2) (layer "F.Cu") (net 3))
 (segment (start 151.85 109.64) (end 153.001 110.791) (width 0.2) (layer "F.Cu") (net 3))
 (segment (start 153.001 112.65676) (end 152.32676 113.331) (width 0.2) (layer "F.Cu") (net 3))
 (segment (start 147.838 133.122) (end 145.338 130.622) (width 0.2) (layer "F.Cu") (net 3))
 (segment (start 111.35 102.025) (end 111.35 100.1355) (width 0.2) (layer "F.Cu") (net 3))
 (segment (start 154.924 126.036) (end 147.838 133.122) (width 0.2) (layer "F.Cu") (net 3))
 (segment (start 151.85 109.64) (end 154.924 112.714) (width 0.2) (layer "F.Cu") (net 3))
 (segment (start 152.32676 113.331) (end 151.37324 113.331) (width 0.2) (layer "F.Cu") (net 3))
 (segment (start 154.924 112.714) (end 154.924 126.036) (width 0.2) (layer "F.Cu") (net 3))
 (segment (start 139.96724 101.925) (end 125.825 101.925) (width 0.2) (layer "F.Cu") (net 3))
 (via (at 123.025 101.9) (size 0.6) (drill 0.3) (layers "F.Cu" "B.Cu") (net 3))
 (via (at 123.45 99.825) (size 0.6) (drill 0.3) (layers "F.Cu" "B.Cu") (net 3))
 (via (at 125.825 101.925) (size 0.6) (drill 0.3) (layers "F.Cu" "B.Cu") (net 3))
 (via (at 120.236732 99.825) (size 0.6) (drill 0.3) (layers "F.Cu" "B.Cu") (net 3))
 (segment (start 86.2125 98.3) (end 106.3785 98.3) (width 0.2) (layer "B.Cu") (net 3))
 (segment (start 123.3875 97.925) (end 123.3875 99.7625) (width 0.2) (layer "B.Cu") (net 3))
 (segment (start 123.3875 99.7625) (end 123.45 99.825) (width 0.2) (layer "B.Cu") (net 3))
 (segment (start 106.3785 98.3) (end 107.529 97.1495) (width 0.2) (layer "B.Cu") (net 3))
 (segment (start 123.3875 97.925) (end 123.5 98.0375) (width 0.2) (layer "B.Cu") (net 3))
 (segment (start 122.311732 101.9) (end 123.025 101.9) (width 0.2) (layer "B.Cu") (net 3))
 (segment (start 125.825 101.925) (end 125.825 100.3625) (width 0.2) (layer "B.Cu") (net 3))
 (segment (start 120.236732 99.825) (end 122.311732 101.9) (width 0.2) (layer "B.Cu") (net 3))
 (segment (start 125.825 100.3625) (end 123.3875 97.925) (width 0.2) (layer "B.Cu") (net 3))
 (segment (start 89.157 127.818) (end 90.427 126.548) (width 0.2) (layer "F.Cu") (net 21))
 (segment (start 77.064 127.818) (end 89.157 127.818) (width 0.2) (layer "F.Cu") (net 21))
 (segment (start 109.517 134.154) (end 128.497 134.154) (width 0.2) (layer "F.Cu") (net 20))
 (segment (start 109.503 134.168) (end 109.517 134.154) (width 0.2) (layer "F.Cu") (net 20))
 (segment (start 90.427 134.168) (end 109.503 134.168) (width 0.2) (layer "F.Cu") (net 20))
 (segment (start 128.497 134.154) (end 128.5 134.157) (width 0.2) (layer "F.Cu") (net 20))
 (segment (start 110.618 105.3185) (end 110.618 133.053) (width 0.2) (layer "B.Cu") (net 20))
 (segment (start 107.529 102.2295) (end 110.618 105.3185) (width 0.2) (layer "B.Cu") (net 20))
 (segment (start 110.618 133.053) (end 109.517 134.154) (width 0.2) (layer "B.Cu") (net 20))
 (segment (start 96.099 127.823) (end 108.228 127.823) (width 0.2) (layer "F.Cu") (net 6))
 (segment (start 108.228 127.823) (end 109.517 126.534) (width 0.2) (layer "F.Cu") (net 6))
 (segment (start 127.21 127.827) (end 128.5 126.537) (width 0.2) (layer "F.Cu") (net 14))
 (segment (start 115.146 127.827) (end 127.21 127.827) (width 0.2) (layer "F.Cu") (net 14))
 (segment (start 100.972 103.2925) (end 92.289 94.6095) (width 0.2) (layer "F.Cu") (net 10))
 (segment (start 110.7355 103.2925) (end 100.972 103.2925) (width 0.2) (layer "F.Cu") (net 10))
 (segment (start 110.738 103.29) (end 110.7355 103.2925) (width 0.2) (layer "F.Cu") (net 10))
 (via (at 110.738 103.29) (size 0.6) (drill 0.3) (layers "F.Cu" "B.Cu") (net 10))
 (segment (start 133.338 128.122) (end 133.338 125.89) (width 0.2) (layer "B.Cu") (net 10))
 (segment (start 133.338 125.89) (end 110.738 103.29) (width 0.2) (layer "B.Cu") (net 10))
 (segment (start 140.095 100.425) (end 119.7 100.425) (width 0.2) (layer "F.Cu") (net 15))
 (segment (start 151.85 112.18) (end 140.095 100.425) (width 0.2) (layer "F.Cu") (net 15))
 (via (at 119.7 100.425) (size 0.6) (drill 0.3) (layers "F.Cu" "B.Cu") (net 15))
 (segment (start 119.7 100.425) (end 119.225 100.425) (width 0.2) (layer "B.Cu") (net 15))
 (segment (start 118.4895 99.6895) (end 107.529 99.6895) (width 0.2) (layer "B.Cu") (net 15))
 (segment (start 119.225 100.425) (end 118.4895 99.6895) (width 0.2) (layer "B.Cu") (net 15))
 (segment (start 111.0125 108.5875) (end 107.391218 108.5875) (width 0.2) (layer "F.Cu") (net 17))
 (segment (start 90.0395 104.7695) (end 92.289 104.7695) (width 0.2) (layer "F.Cu") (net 17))
 (segment (start 111.55 109.125) (end 111.0125 108.5875) (width 0.2) (layer "F.Cu") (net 17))
 (segment (start 151.85 117.26) (end 122.635 117.26) (width 0.2) (layer "F.Cu") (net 17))
 (segment (start 91.6065 104.7695) (end 92.289 104.7695) (width 0.2) (layer "F.Cu") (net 17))
 (segment (start 122.635 117.26) (end 115.65 110.275) (width 0.2) (layer "F.Cu") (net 17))
 (via (at 107.391218 108.5875) (size 0.6) (drill 0.3) (layers "F.Cu" "B.Cu") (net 17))
 (via (at 111.55 109.125) (size 0.6) (drill 0.3) (layers "F.Cu" "B.Cu") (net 17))
 (via (at 115.65 110.275) (size 0.6) (drill 0.3) (layers "F.Cu" "B.Cu") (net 17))
 (segment (start 103.1945 104.7695) (end 92.289 104.7695) (width 0.2) (layer "B.Cu") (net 17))
 (segment (start 115.65 110.275) (end 114.425 109.05) (width 0.2) (layer "B.Cu") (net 17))
 (segment (start 107.391218 108.5875) (end 107.0125 108.5875) (width 0.2) (layer "B.Cu") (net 17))
 (segment (start 114.425 109.05) (end 111.625 109.05) (width 0.2) (layer "B.Cu") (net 17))
 (segment (start 111.625 109.05) (end 111.55 109.125) (width 0.2) (layer "B.Cu") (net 17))
 (segment (start 107.0125 108.5875) (end 103.1945 104.7695) (width 0.2) (layer "B.Cu") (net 17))
 (segment (start 93.766 101.1665) (end 92.289 99.6895) (width 0.2) (layer "B.Cu") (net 12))
 (segment (start 120.8825 101.1665) (end 93.766 101.1665) (width 0.2) (layer "B.Cu") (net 12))
 (segment (start 147.838 128.122) (end 120.8825 101.1665) (width 0.2) (layer "B.Cu") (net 12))
 (segment (start 133.338 133.122) (end 129.601 129.385) (width 0.2) (layer "F.Cu") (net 11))
 (segment (start 111.803 118.388) (end 105.413 111.998) (width 0.2) (layer "F.Cu") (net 11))
 (segment (start 129.601 129.385) (end 129.601 126.08095) (width 0.2) (layer "F.Cu") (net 11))
 (segment (start 105.413 111.998) (end 104.41 111.998) (width 0.2) (layer "F.Cu") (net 11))
 (segment (start 125.60505 122.085) (end 122.767 122.085) (width 0.2) (layer "F.Cu") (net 11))
 (segment (start 129.601 126.08095) (end 125.60505 122.085) (width 0.2) (layer "F.Cu") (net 11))
 (segment (start 101.403 106.2635) (end 92.289 97.1495) (width 0.2) (layer "F.Cu") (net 11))
 (segment (start 101.403 110.996) (end 101.403 106.2635) (width 0.2) (layer "F.Cu") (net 11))
 (via (at 122.767 122.085) (size 0.6) (drill 0.3) (layers "F.Cu" "B.Cu") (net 11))
 (via (at 111.803 118.388) (size 0.6) (drill 0.3) (layers "F.Cu" "B.Cu") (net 11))
 (via (at 104.41 111.998) (size 0.6) (drill 0.3) (layers "F.Cu" "B.Cu") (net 11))
 (via (at 101.403 110.996) (size 0.6) (drill 0.3) (layers "F.Cu" "B.Cu") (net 11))
 (segment (start 122.767 122.085) (end 115.5 122.085) (width 0.2) (layer "B.Cu") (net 11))
 (segment (start 102.405 111.998) (end 101.403 110.996) (width 0.2) (layer "B.Cu") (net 11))
 (segment (start 104.41 111.998) (end 102.405 111.998) (width 0.2) (layer "B.Cu") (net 11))
 (segment (start 115.5 122.085) (end 111.803 118.388) (width 0.2) (layer "B.Cu") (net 11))
 (segment (start 91.213 152.148) (end 91.213 137.156) (width 0.2) (layer "F.Cu") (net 19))
 (segment (start 109.436 153.249) (end 109.659 153.026) (width 0.2) (layer "F.Cu") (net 19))
 (segment (start 109.659 153.026) (end 128.591 153.026) (width 0.2) (layer "F.Cu") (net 19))
 (segment (start 128.591 153.026) (end 128.597 153.02) (width 0.2) (layer "F.Cu") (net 19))
 (segment (start 90.112 153.249) (end 91.213 152.148) (width 0.2) (layer "F.Cu") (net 19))
 (segment (start 92.289 126.24305) (end 92.289 109.8495) (width 0.2) (layer "F.Cu") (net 19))
 (segment (start 89.326 135.269) (end 89.326 129.20605) (width 0.2) (layer "F.Cu") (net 19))
 (segment (start 89.326 129.20605) (end 92.289 126.24305) (width 0.2) (layer "F.Cu") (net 19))
 (segment (start 90.112 153.249) (end 109.436 153.249) (width 0.2) (layer "F.Cu") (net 19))
 (segment (start 91.213 137.156) (end 89.326 135.269) (width 0.2) (layer "F.Cu") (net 19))
 (segment (start 88.894 146.847) (end 90.112 145.629) (width 0.2) (layer "F.Cu") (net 8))
 (segment (start 77.071 146.847) (end 88.894 146.847) (width 0.2) (layer "F.Cu") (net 8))
 (segment (start 108.22 146.845) (end 109.659 145.406) (width 0.2) (layer "F.Cu") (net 18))
 (segment (start 96.102 146.845) (end 108.22 146.845) (width 0.2) (layer "F.Cu") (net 18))
 (segment (start 115.205 146.899) (end 127.098 146.899) (width 0.2) (layer "F.Cu") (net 22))
 (segment (start 127.098 146.899) (end 128.597 145.4) (width 0.2) (layer "F.Cu") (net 22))
 (segment (start 90.177 118.515) (end 90.91 118.515) (width 0.2) (layer "F.Cu") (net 7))
 (segment (start 83.414 125.278) (end 90.177 118.515) (width 0.2) (layer "F.Cu") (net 7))
 (via (at 90.91 118.515) (size 0.6) (drill 0.3) (layers "F.Cu" "B.Cu") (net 7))
 (segment (start 83.414 125.278) (end 83.414 144.3) (width 0.2) (layer "B.Cu") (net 7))
 (segment (start 83.414 144.3) (end 83.421 144.307) (width 0.2) (layer "B.Cu") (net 7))
 (segment (start 99.5755 109.8495) (end 107.529 109.8495) (width 0.2) (layer "B.Cu") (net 7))
 (segment (start 90.91 118.515) (end 99.5755 109.8495) (width 0.2) (layer "B.Cu") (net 7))
 (segment (start 102.449 112.3895) (end 107.529 107.3095) (width 0.2) (layer "F.Cu") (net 5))
 (segment (start 102.449 125.283) (end 102.449 112.3895) (width 0.2) (layer "F.Cu") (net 5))
 (segment (start 102.449 144.302) (end 102.452 144.305) (width 0.2) (layer "B.Cu") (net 5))
 (segment (start 102.449 125.283) (end 102.449 144.302) (width 0.2) (layer "B.Cu") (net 5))
 (segment (start 108.60663 104.7695) (end 121.496 117.65887) (width 0.2) (layer "F.Cu") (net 13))
 (segment (start 107.529 104.7695) (end 108.60663 104.7695) (width 0.2) (layer "F.Cu") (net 13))
 (segment (start 121.496 117.65887) (end 121.496 125.287) (width 0.2) (layer "F.Cu") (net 13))
 (segment (start 121.496 125.287) (end 121.496 144.3) (width 0.2) (layer "B.Cu") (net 13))
 (segment (start 121.496 144.3) (end 121.555 144.359) (width 0.2) (layer "B.Cu") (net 13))
 (segment (start 111.5 111.5) (end 105.775 111.5) (width 0.2) (layer "F.Cu") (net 16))
 (segment (start 151.85 114.72) (end 148.655 111.525) (width 0.2) (layer "F.Cu") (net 16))
 (segment (start 105.775 111.5) (end 105.25 110.975) (width 0.2) (layer "F.Cu") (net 16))
 (segment (start 100.275 110.4495) (end 97.135 107.3095) (width 0.2) (layer "F.Cu") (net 16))
 (segment (start 148.655 111.525) (end 118.1 111.525) (width 0.2) (layer "F.Cu") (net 16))
 (segment (start 97.135 107.3095) (end 92.289 107.3095) (width 0.2) (layer "F.Cu") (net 16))
 (segment (start 90.0395 107.3095) (end 92.289 107.3095) (width 0.2) (layer "F.Cu") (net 16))
 (via (at 118.1 111.525) (size 0.6) (drill 0.3) (layers "F.Cu" "B.Cu") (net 16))
 (via (at 100.275 110.4495) (size 0.6) (drill 0.3) (layers "F.Cu" "B.Cu") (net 16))
 (via (at 105.25 110.975) (size 0.6) (drill 0.3) (layers "F.Cu" "B.Cu") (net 16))
 (via (at 111.5 111.5) (size 0.6) (drill 0.3) (layers "F.Cu" "B.Cu") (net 16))
 (segment (start 105.25 110.975) (end 104.67 110.395) (width 0.2) (layer "B.Cu") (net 16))
 (segment (start 100.3295 110.395) (end 100.275 110.4495) (width 0.2) (layer "B.Cu") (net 16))
 (segment (start 104.67 110.395) (end 100.3295 110.395) (width 0.2) (layer "B.Cu") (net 16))
 (segment (start 118.1 111.525) (end 111.525 111.525) (width 0.2) (layer "B.Cu") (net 16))
 (segment (start 111.525 111.525) (end 111.5 111.5) (width 0.2) (layer "B.Cu") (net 16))
 (segment (start 88 98.7755) (end 91.454 102.2295) (width 0.2) (layer "F.Cu") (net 4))
 (segment (start 88 97.6) (end 88 98.7755) (width 0.2) (layer "F.Cu") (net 4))
 (segment (start 91.454 102.2295) (end 92.289 102.2295) (width 0.2) (layer "F.Cu") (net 4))
 (via (at 88 97.6) (size 0.6) (drill 0.3) (layers "F.Cu" "B.Cu") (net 4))
 (segment (start 86.2125 96.8) (end 87.2 96.8) (width 0.2) (layer "B.Cu") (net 4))
 (segment (start 87.2 96.8) (end 88 97.6) (width 0.2) (layer "B.Cu") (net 4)))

